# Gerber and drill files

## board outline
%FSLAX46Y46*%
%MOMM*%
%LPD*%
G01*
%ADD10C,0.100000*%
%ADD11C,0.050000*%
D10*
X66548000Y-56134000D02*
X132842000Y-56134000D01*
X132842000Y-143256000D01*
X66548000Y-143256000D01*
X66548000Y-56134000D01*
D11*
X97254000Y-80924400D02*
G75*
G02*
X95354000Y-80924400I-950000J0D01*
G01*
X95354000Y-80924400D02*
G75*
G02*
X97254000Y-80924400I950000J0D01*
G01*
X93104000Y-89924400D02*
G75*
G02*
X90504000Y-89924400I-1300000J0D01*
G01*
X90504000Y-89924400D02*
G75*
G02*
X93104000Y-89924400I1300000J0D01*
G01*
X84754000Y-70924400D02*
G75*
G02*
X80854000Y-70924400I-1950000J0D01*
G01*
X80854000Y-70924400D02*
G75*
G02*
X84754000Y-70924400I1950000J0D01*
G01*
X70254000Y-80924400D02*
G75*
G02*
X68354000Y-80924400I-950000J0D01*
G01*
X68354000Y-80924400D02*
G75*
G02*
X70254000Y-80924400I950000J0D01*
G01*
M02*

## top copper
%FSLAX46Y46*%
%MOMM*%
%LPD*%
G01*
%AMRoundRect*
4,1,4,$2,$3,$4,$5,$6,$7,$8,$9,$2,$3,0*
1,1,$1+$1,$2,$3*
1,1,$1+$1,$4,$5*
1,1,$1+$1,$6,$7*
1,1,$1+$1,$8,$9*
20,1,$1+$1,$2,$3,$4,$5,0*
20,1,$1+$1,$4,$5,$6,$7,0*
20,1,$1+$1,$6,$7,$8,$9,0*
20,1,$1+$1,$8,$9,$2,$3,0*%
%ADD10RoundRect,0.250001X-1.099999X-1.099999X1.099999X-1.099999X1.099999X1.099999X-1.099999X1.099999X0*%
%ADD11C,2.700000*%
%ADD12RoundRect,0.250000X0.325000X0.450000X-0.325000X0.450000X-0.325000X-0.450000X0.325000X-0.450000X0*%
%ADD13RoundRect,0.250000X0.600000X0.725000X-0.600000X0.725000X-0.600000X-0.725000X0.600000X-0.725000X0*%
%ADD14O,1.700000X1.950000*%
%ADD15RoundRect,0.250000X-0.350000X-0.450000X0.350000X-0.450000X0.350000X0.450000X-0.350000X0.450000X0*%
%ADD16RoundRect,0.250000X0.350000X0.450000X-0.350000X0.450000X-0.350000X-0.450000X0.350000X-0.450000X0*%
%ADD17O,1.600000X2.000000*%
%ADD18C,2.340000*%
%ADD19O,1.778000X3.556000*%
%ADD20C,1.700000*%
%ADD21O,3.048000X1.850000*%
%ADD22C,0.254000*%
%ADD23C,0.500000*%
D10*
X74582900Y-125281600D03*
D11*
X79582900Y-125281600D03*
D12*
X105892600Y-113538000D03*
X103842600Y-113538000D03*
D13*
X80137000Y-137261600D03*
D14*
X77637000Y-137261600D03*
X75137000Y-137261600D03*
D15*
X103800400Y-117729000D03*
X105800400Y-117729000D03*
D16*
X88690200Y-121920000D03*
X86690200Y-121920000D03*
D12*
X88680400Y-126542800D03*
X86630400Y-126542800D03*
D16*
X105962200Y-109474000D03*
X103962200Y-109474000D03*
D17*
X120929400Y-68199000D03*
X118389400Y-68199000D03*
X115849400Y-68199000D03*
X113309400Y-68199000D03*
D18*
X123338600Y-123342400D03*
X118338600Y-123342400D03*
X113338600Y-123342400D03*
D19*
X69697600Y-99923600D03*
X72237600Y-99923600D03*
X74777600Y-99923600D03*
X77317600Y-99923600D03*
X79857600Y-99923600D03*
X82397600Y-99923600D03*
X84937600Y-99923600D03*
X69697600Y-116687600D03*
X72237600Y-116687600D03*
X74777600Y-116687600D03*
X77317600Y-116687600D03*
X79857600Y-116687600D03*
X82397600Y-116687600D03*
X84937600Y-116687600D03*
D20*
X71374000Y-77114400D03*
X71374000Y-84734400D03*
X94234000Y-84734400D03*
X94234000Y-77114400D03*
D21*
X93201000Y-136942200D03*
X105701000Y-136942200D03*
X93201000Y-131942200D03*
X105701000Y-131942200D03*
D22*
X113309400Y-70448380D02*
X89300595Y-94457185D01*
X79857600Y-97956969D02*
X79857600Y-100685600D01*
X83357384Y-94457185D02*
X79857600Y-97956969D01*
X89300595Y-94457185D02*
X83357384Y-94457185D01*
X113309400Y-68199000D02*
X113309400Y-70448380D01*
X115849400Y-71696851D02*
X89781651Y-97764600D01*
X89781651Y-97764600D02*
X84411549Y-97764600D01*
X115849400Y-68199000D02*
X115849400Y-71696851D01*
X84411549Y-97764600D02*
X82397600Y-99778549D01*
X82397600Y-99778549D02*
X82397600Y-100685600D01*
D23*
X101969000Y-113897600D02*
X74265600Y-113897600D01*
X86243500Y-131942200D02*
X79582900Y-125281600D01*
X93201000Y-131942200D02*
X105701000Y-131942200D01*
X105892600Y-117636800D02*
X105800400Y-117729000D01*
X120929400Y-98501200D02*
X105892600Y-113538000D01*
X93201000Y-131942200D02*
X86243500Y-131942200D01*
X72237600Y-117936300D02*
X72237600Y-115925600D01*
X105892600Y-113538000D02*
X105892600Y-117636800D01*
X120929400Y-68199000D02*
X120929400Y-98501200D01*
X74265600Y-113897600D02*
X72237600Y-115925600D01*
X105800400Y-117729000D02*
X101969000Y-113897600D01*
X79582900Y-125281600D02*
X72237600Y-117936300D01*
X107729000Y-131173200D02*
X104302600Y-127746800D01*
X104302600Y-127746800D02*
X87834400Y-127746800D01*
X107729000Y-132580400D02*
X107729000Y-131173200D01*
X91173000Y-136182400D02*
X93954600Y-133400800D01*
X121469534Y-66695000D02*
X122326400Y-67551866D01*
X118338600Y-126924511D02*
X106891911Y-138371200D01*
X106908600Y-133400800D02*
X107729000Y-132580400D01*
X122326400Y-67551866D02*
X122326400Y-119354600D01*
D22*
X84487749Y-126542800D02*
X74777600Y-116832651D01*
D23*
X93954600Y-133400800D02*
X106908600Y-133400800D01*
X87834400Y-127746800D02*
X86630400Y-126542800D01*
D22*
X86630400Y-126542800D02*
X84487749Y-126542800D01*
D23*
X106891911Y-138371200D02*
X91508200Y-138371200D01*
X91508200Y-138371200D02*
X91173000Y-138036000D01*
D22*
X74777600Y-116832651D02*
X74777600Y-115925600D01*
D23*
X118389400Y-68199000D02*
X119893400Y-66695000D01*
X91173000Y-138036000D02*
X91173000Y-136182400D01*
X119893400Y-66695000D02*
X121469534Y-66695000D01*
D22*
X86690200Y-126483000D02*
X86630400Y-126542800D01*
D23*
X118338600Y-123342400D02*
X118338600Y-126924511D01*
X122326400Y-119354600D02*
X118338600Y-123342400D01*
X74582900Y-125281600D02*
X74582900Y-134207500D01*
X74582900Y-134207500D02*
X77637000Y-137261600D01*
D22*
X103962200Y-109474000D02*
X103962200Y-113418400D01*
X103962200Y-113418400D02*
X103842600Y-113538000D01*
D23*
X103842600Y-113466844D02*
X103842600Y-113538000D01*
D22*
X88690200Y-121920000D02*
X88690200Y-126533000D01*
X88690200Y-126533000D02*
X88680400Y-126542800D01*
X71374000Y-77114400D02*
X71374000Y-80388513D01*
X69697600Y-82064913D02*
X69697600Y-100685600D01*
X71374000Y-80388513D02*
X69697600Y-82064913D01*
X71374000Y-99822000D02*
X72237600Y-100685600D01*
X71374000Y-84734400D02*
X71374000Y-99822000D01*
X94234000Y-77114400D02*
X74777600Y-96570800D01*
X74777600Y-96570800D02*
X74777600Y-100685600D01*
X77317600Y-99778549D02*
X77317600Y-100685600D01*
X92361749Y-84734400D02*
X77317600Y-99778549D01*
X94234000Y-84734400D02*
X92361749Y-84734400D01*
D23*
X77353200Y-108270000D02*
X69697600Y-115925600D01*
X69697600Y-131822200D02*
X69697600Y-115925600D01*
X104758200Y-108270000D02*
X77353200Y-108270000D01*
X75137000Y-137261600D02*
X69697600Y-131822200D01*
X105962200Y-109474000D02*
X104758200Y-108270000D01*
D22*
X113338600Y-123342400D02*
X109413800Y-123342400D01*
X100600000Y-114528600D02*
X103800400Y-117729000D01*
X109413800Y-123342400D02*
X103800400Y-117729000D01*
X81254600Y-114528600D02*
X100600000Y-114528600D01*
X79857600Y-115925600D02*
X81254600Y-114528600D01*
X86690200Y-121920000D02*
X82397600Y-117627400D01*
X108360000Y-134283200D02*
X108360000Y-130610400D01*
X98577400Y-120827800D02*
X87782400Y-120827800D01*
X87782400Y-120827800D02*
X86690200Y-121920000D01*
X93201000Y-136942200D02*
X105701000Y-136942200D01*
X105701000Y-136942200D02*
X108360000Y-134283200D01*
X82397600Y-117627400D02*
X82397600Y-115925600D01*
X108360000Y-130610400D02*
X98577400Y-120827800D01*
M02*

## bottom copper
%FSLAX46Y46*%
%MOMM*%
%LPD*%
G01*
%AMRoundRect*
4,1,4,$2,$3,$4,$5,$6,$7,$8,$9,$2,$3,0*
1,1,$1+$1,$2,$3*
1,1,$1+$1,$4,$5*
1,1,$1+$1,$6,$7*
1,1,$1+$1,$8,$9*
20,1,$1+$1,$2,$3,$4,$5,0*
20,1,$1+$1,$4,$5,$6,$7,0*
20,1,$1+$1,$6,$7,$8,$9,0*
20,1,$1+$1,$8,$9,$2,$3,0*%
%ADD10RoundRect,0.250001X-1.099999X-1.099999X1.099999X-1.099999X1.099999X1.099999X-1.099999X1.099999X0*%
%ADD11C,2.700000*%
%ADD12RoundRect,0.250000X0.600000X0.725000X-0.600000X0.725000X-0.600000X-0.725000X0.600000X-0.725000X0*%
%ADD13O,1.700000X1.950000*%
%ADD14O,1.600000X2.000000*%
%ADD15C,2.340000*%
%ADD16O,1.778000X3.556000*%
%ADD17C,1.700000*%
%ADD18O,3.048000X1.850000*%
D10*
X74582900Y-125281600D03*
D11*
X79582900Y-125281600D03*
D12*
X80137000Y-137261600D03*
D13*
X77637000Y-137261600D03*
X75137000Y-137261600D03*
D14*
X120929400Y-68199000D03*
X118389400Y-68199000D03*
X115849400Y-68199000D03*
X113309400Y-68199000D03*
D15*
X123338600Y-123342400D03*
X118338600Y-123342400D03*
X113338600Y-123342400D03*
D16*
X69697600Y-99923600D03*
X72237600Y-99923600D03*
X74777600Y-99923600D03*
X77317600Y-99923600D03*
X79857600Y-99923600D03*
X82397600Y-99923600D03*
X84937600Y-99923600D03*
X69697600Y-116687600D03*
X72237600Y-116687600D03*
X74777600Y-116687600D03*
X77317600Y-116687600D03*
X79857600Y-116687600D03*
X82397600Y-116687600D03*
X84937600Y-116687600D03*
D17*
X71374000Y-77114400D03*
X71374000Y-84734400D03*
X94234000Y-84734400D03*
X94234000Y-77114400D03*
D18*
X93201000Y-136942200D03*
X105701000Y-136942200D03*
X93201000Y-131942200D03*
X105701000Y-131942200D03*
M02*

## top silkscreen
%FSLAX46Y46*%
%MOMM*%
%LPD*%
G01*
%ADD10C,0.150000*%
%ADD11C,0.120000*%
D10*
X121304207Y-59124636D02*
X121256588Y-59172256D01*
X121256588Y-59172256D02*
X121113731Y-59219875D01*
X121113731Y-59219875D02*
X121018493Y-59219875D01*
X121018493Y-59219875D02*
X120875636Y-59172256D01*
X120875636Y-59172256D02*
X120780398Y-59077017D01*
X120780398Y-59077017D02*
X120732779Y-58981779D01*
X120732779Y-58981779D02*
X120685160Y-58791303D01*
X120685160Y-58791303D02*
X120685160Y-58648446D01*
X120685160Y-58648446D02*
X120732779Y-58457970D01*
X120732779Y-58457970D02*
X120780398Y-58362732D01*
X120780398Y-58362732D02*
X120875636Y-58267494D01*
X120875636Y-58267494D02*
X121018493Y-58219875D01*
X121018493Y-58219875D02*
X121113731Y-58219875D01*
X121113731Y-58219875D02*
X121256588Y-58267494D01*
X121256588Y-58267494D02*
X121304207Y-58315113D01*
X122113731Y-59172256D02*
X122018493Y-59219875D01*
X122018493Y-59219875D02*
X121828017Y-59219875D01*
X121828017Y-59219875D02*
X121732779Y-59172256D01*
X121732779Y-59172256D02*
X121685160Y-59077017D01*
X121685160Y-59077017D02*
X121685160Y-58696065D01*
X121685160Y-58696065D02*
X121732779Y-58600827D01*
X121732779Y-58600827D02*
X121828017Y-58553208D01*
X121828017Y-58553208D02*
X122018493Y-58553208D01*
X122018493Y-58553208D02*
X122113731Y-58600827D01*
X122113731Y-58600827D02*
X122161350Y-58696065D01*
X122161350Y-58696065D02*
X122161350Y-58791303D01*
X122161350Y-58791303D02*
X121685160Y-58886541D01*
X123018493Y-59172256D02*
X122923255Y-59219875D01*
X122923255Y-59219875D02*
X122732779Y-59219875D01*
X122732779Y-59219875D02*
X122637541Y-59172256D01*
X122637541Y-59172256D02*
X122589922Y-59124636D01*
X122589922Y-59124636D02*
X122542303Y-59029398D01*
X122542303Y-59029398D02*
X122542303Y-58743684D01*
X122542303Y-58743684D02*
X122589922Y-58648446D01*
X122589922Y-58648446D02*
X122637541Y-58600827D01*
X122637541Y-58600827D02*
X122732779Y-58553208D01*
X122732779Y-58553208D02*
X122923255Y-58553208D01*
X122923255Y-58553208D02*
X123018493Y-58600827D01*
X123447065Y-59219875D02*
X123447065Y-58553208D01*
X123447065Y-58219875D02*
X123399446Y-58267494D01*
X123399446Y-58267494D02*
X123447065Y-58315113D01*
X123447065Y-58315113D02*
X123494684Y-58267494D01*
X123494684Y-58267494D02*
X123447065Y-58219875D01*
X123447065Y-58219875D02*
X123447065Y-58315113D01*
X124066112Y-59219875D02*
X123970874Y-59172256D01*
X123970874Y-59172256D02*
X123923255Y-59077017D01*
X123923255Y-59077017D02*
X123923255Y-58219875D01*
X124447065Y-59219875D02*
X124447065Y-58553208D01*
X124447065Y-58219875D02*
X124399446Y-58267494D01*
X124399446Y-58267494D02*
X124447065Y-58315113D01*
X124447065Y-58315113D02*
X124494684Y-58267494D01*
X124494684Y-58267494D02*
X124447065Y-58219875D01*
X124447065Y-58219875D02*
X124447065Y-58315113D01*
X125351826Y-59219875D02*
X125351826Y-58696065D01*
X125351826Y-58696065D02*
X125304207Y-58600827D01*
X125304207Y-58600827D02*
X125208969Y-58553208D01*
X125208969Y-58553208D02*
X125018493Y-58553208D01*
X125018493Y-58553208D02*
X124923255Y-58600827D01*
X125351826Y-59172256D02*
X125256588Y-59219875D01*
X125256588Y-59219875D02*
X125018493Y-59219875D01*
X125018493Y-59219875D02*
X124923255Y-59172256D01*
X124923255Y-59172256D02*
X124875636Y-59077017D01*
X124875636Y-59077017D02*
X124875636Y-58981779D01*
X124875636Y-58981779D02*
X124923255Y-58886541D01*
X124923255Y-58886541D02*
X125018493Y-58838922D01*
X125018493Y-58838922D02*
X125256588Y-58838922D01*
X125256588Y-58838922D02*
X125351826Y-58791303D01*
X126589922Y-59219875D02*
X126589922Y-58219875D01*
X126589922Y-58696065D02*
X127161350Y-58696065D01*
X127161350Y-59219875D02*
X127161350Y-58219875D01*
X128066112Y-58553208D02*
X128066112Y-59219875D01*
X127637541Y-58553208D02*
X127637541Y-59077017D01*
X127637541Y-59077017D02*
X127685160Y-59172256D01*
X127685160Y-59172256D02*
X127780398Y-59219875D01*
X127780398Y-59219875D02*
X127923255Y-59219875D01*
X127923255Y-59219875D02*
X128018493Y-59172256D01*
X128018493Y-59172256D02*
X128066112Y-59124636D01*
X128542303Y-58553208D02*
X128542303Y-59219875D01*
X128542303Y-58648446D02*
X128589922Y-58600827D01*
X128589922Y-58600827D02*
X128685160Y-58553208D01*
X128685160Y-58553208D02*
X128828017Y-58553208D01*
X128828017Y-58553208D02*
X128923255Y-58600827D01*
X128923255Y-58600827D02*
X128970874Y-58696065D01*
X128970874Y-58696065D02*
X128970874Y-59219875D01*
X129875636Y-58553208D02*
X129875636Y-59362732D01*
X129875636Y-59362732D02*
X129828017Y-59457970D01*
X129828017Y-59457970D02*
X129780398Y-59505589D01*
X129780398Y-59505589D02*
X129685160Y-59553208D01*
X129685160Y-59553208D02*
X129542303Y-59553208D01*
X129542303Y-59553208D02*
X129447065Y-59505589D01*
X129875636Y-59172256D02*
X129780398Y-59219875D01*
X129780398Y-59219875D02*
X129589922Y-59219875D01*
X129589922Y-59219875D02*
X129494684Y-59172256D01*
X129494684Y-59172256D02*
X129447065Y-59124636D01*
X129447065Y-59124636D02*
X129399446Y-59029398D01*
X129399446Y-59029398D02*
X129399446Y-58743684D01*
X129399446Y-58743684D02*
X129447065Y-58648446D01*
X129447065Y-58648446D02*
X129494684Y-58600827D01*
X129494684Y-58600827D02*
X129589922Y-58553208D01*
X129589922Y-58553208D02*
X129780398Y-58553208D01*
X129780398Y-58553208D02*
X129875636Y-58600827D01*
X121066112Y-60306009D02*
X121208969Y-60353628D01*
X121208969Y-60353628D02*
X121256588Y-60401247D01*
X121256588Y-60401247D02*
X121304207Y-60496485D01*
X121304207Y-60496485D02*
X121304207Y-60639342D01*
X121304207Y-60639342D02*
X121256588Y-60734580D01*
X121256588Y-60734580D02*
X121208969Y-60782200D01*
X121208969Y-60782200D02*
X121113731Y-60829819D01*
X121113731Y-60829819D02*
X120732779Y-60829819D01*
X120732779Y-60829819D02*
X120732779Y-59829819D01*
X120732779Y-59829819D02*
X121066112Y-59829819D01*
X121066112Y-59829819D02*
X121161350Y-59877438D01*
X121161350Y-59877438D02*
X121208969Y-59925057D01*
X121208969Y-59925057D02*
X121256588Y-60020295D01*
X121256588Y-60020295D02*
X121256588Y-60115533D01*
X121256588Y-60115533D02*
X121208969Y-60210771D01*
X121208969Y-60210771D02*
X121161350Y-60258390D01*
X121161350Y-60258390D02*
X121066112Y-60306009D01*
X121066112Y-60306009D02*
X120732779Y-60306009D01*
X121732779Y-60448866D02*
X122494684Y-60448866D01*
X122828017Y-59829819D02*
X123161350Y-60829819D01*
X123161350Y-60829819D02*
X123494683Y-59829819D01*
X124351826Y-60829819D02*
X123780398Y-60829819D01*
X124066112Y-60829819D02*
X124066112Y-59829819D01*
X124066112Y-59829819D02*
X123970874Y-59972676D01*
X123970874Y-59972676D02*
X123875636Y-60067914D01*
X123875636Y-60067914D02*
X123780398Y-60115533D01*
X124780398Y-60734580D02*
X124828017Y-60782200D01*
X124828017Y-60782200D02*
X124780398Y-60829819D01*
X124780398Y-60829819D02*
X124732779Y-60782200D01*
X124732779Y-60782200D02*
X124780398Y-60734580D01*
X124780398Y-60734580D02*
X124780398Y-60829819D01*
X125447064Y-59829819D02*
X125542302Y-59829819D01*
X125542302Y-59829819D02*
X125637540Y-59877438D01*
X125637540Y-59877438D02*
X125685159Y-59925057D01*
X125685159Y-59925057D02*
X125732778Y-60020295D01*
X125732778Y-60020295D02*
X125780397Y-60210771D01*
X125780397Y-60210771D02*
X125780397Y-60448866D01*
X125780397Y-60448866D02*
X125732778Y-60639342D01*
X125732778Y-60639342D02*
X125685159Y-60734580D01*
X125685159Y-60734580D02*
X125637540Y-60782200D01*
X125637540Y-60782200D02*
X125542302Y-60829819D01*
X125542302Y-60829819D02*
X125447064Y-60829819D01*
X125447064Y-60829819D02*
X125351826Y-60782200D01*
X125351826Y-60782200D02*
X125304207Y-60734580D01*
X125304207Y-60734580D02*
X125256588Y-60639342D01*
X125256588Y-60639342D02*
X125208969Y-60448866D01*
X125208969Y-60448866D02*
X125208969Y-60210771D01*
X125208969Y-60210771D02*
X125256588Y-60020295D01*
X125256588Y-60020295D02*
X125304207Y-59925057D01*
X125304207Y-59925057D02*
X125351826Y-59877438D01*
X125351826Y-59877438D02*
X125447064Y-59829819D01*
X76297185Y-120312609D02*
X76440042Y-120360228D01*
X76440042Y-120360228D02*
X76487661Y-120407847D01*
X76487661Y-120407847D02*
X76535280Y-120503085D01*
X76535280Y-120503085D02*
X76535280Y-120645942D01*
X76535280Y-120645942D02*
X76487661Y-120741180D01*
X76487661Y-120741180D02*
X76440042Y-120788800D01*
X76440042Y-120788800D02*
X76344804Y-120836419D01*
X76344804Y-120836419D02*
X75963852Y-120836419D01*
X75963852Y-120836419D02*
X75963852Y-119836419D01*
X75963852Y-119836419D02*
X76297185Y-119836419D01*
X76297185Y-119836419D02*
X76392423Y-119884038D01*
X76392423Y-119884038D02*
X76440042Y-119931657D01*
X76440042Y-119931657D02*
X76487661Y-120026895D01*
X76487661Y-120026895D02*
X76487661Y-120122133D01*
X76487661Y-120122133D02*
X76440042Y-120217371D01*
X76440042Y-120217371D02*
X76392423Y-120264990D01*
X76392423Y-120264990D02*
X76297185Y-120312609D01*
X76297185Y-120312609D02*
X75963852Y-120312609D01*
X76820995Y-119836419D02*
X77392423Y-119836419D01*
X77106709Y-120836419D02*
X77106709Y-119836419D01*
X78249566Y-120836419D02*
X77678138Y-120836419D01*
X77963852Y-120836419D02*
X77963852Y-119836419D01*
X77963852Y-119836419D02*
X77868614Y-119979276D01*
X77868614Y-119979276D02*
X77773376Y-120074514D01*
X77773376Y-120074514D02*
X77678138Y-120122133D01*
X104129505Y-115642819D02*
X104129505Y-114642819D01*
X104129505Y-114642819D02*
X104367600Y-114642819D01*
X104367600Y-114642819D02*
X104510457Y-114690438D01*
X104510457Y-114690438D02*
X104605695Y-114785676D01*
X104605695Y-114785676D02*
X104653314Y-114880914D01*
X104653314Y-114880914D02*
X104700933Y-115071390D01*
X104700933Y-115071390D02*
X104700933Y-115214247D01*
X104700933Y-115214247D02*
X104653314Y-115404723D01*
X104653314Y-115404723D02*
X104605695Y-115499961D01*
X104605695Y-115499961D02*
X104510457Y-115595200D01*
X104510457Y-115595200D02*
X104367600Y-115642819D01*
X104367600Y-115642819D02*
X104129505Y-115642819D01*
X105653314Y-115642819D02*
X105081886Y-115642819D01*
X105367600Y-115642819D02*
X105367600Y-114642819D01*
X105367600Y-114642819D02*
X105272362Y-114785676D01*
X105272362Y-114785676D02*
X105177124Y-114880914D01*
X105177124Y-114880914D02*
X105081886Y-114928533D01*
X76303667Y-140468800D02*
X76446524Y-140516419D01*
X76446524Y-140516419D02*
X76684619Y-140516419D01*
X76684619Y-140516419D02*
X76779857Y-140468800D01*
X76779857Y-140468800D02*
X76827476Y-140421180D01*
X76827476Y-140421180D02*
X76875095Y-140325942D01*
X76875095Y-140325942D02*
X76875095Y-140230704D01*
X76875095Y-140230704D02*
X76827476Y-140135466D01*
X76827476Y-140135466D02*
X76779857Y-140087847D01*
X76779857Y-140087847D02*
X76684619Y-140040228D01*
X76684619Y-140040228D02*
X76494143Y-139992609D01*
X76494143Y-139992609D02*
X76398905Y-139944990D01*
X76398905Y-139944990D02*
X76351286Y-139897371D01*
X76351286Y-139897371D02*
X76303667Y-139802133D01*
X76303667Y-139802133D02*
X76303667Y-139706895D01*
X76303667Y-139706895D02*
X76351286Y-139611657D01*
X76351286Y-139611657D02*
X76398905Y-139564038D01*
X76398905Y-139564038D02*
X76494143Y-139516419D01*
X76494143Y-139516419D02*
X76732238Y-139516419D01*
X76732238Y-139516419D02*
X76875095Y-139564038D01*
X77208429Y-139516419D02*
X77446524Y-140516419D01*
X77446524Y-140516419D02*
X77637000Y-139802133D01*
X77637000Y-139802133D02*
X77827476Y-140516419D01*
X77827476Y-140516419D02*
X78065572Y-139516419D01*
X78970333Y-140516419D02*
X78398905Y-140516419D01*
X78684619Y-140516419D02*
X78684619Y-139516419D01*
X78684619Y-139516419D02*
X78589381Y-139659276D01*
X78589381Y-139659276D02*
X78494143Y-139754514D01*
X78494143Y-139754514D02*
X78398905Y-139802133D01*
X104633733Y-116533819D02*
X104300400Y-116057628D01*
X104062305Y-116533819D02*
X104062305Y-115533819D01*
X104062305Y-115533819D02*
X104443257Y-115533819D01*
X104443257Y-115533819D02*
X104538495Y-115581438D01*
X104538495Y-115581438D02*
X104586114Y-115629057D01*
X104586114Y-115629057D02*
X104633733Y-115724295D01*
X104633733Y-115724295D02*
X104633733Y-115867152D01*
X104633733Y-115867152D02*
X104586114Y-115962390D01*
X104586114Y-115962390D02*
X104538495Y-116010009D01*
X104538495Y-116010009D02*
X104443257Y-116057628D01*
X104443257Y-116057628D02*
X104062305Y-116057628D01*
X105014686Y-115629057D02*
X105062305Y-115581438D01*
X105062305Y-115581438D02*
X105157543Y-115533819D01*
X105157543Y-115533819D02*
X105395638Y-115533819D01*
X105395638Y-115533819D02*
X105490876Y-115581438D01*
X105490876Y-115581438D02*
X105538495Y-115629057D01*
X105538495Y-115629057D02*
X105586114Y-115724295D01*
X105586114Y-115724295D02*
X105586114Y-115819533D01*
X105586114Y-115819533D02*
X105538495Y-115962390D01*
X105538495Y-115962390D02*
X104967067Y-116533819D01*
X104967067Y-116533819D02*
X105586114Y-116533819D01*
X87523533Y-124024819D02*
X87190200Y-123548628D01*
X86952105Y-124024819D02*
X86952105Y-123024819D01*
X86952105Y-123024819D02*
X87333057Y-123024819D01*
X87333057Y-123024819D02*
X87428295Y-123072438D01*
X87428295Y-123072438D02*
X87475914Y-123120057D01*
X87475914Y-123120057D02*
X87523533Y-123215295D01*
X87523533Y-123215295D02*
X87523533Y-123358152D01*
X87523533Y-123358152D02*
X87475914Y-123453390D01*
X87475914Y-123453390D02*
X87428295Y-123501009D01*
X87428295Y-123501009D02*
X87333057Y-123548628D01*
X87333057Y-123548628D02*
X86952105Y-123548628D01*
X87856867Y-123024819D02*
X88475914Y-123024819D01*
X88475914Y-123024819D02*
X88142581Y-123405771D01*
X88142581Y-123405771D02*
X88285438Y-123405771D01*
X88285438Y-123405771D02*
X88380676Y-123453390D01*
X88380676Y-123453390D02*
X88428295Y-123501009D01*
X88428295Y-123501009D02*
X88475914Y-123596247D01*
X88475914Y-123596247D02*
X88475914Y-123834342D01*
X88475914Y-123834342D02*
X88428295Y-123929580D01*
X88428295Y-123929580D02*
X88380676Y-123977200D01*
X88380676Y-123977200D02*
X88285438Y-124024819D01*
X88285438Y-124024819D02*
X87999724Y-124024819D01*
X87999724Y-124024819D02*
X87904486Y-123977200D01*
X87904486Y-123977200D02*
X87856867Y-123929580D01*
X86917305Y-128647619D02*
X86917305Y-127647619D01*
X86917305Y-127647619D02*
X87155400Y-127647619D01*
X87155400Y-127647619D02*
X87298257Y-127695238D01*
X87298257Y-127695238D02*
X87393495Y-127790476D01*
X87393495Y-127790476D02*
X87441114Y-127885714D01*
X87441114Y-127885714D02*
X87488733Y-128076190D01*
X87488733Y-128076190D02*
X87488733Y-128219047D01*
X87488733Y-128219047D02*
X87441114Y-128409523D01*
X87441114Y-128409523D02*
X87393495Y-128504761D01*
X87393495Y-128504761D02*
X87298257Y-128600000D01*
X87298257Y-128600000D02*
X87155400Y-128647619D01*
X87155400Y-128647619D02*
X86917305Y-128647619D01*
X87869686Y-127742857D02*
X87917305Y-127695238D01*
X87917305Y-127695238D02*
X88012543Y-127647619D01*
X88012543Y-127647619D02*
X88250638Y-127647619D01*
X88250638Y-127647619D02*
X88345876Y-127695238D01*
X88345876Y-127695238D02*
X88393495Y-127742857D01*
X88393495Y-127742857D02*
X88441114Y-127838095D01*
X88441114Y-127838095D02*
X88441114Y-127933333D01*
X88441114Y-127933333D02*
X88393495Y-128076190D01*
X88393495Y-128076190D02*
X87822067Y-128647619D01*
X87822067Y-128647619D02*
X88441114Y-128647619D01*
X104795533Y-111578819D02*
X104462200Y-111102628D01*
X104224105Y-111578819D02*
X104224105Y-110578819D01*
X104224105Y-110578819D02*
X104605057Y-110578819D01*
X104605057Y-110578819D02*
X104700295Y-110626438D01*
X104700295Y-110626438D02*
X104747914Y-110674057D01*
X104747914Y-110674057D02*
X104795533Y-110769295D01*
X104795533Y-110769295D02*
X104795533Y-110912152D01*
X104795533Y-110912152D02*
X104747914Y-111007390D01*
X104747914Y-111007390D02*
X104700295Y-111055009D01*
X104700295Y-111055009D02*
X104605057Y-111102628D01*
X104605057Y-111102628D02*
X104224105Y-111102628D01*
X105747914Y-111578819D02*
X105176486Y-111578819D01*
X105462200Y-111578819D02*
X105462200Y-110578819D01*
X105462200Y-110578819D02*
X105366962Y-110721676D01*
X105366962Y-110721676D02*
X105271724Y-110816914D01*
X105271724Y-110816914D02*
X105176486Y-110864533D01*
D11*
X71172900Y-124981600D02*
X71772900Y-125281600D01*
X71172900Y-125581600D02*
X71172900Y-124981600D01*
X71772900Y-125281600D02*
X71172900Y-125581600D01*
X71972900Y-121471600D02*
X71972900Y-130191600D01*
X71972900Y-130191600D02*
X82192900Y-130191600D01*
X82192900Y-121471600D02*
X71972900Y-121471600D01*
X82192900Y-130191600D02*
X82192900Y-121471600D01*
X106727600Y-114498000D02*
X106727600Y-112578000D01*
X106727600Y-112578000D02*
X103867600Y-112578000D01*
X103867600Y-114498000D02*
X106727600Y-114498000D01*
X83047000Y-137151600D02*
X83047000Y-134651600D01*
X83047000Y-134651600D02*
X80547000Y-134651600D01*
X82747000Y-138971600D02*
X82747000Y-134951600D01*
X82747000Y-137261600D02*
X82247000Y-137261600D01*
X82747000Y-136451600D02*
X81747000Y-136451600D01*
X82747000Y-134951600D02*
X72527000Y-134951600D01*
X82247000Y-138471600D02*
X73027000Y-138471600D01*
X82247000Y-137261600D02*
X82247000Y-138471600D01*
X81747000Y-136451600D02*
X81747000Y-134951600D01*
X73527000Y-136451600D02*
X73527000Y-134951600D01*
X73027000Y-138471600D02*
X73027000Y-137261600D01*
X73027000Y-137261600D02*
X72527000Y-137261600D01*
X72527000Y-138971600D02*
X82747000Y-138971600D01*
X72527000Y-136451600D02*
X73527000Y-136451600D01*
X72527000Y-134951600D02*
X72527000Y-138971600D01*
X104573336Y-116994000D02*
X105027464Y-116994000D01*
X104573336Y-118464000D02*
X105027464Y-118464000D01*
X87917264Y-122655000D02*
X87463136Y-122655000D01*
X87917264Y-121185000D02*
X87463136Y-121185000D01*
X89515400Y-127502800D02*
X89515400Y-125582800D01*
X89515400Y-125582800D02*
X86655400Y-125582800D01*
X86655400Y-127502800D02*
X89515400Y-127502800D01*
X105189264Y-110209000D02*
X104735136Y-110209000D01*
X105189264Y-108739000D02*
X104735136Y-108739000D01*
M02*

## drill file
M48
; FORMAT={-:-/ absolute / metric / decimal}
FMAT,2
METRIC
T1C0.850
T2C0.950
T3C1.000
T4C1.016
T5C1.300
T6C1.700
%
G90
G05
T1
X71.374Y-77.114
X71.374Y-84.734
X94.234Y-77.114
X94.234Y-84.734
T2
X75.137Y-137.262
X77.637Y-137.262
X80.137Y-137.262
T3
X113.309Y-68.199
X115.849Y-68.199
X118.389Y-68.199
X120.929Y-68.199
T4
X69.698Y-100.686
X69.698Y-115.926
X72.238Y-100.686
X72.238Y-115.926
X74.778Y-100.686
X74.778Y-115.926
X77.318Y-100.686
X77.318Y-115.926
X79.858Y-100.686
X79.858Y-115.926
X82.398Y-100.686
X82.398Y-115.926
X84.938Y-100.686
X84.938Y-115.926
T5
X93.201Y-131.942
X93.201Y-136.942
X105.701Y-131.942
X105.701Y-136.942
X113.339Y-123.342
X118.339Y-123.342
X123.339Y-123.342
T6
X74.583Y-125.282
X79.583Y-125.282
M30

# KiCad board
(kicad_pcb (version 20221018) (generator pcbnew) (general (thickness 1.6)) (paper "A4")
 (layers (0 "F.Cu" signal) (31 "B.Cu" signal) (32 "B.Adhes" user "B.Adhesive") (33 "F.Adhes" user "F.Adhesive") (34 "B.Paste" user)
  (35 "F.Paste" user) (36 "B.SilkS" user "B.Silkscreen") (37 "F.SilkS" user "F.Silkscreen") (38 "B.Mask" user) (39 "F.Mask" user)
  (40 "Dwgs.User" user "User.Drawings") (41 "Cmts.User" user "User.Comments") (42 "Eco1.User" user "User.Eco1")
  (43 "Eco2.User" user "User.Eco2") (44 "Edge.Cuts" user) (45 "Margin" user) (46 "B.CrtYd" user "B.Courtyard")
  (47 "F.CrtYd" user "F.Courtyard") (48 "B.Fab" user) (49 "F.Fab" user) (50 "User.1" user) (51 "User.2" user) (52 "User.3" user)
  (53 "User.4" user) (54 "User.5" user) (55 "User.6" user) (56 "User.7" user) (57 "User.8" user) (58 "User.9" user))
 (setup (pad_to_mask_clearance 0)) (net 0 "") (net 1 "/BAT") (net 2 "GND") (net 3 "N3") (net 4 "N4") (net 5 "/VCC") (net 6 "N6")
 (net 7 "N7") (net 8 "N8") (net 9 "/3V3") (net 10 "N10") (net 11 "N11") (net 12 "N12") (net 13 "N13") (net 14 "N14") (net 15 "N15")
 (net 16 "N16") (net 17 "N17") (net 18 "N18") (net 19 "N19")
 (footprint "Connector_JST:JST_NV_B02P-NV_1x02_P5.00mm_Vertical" (layer "F.Cu") (at 74.5829 125.2816)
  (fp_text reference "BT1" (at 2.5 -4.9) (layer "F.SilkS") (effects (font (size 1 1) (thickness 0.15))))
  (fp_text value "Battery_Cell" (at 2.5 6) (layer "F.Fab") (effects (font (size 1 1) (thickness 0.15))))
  (fp_line (start -3.41 -0.3) (end -2.81 0) (stroke (width 0.12) (type solid)) (layer "F.SilkS"))
  (fp_line (start -3.41 0.3) (end -3.41 -0.3) (stroke (width 0.12) (type solid)) (layer "F.SilkS"))
  (fp_line (start -2.81 0) (end -3.41 0.3) (stroke (width 0.12) (type solid)) (layer "F.SilkS"))
  (fp_line (start -2.61 -3.81) (end -2.61 4.91) (stroke (width 0.12) (type solid)) (layer "F.SilkS"))
  (fp_line (start -2.61 4.91) (end 7.61 4.91) (stroke (width 0.12) (type solid)) (layer "F.SilkS"))
  (fp_line (start 7.61 -3.81) (end -2.61 -3.81) (stroke (width 0.12) (type solid)) (layer "F.SilkS"))
  (fp_line (start 7.61 4.91) (end 7.61 -3.81) (stroke (width 0.12) (type solid)) (layer "F.SilkS"))
  (pad "1" thru_hole roundrect (at 0 0) (size 2.7 2.7) (drill 1.7) (layers "*.Cu" "*.Mask") (roundrect_rratio 0.09259296296) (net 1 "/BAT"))
  (pad "2" thru_hole circle (at 5 0) (size 2.7 2.7) (drill 1.7) (layers "*.Cu" "*.Mask") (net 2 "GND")))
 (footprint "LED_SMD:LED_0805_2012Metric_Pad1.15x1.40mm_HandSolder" (layer "F.Cu") (at 104.8676 113.538 180)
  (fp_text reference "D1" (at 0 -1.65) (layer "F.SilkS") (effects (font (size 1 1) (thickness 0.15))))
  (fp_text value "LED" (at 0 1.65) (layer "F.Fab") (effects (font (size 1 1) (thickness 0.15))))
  (fp_line (start -1.86 -0.96) (end -1.86 0.96) (stroke (width 0.12) (type solid)) (layer "F.SilkS"))
  (fp_line (start -1.86 0.96) (end 1 0.96) (stroke (width 0.12) (type solid)) (layer "F.SilkS"))
  (fp_line (start 1 -0.96) (end -1.86 -0.96) (stroke (width 0.12) (type solid)) (layer "F.SilkS"))
  (pad "1" smd roundrect (at -1.025 0 180) (size 1.15 1.4) (layers "F.Cu" "F.Paste" "F.Mask") (roundrect_rratio 0.2173913043) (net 2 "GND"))
  (pad "2" smd roundrect (at 1.025 0 180) (size 1.15 1.4) (layers "F.Cu" "F.Paste" "F.Mask") (roundrect_rratio 0.2173913043) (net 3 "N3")))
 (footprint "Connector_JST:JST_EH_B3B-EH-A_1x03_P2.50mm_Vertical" (layer "F.Cu") (at 80.137 137.2616 180)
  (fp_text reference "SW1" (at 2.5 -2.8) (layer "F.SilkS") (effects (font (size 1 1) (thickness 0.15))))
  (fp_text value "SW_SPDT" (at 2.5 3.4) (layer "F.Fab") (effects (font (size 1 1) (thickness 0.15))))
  (fp_line (start -2.91 0.11) (end -2.91 2.61) (stroke (width 0.12) (type solid)) (layer "F.SilkS"))
  (fp_line (start -2.91 2.61) (end -0.41 2.61) (stroke (width 0.12) (type solid)) (layer "F.SilkS"))
  (fp_line (start -2.61 -1.71) (end -2.61 2.31) (stroke (width 0.12) (type solid)) (layer "F.SilkS"))
  (fp_line (start -2.61 0) (end -2.11 0) (stroke (width 0.12) (type solid)) (layer "F.SilkS"))
  (fp_line (start -2.61 0.81) (end -1.61 0.81) (stroke (width 0.12) (type solid)) (layer "F.SilkS"))
  (fp_line (start -2.61 2.31) (end 7.61 2.31) (stroke (width 0.12) (type solid)) (layer "F.SilkS"))
  (fp_line (start -2.11 -1.21) (end 7.11 -1.21) (stroke (width 0.12) (type solid)) (layer "F.SilkS"))
  (fp_line (start -2.11 0) (end -2.11 -1.21) (stroke (width 0.12) (type solid)) (layer "F.SilkS"))
  (fp_line (start -1.61 0.81) (end -1.61 2.31) (stroke (width 0.12) (type solid)) (layer "F.SilkS"))
  (fp_line (start 6.61 0.81) (end 6.61 2.31) (stroke (width 0.12) (type solid)) (layer "F.SilkS"))
  (fp_line (start 7.11 -1.21) (end 7.11 0) (stroke (width 0.12) (type solid)) (layer "F.SilkS"))
  (fp_line (start 7.11 0) (end 7.61 0) (stroke (width 0.12) (type solid)) (layer "F.SilkS"))
  (fp_line (start 7.61 -1.71) (end -2.61 -1.71) (stroke (width 0.12) (type solid)) (layer "F.SilkS"))
  (fp_line (start 7.61 0.81) (end 6.61 0.81) (stroke (width 0.12) (type solid)) (layer "F.SilkS"))
  (fp_line (start 7.61 2.31) (end 7.61 -1.71) (stroke (width 0.12) (type solid)) (layer "F.SilkS"))
  (pad "1" thru_hole roundrect (at 0 0 180) (size 1.7 1.95) (drill 0.95) (layers "*.Cu" "*.Mask") (roundrect_rratio 0.1470588235)
   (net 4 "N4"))
  (pad "2" thru_hole oval (at 2.5 0 180) (size 1.7 1.95) (drill 0.95) (layers "*.Cu" "*.Mask") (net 1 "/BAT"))
  (pad "3" thru_hole oval (at 5 0 180) (size 1.7 1.95) (drill 0.95) (layers "*.Cu" "*.Mask") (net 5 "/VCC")))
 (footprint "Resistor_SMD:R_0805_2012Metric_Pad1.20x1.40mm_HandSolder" (layer "F.Cu") (at 104.8004 117.729)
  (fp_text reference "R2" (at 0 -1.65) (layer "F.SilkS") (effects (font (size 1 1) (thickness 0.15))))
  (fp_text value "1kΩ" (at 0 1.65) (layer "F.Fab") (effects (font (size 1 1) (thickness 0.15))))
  (fp_line (start -0.227064 -0.735) (end 0.227064 -0.735) (stroke (width 0.12) (type solid)) (layer "F.SilkS"))
  (fp_line (start -0.227064 0.735) (end 0.227064 0.735) (stroke (width 0.12) (type solid)) (layer "F.SilkS"))
  (pad "1" smd roundrect (at -1 0) (size 1.2 1.4) (layers "F.Cu" "F.Paste" "F.Mask") (roundrect_rratio 0.2083333333) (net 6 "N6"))
  (pad "2" smd roundrect (at 1 0) (size 1.2 1.4) (layers "F.Cu" "F.Paste" "F.Mask") (roundrect_rratio 0.2083333333) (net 2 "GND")))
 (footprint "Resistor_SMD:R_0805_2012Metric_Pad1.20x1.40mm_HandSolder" (layer "F.Cu") (at 87.6902 121.92 180)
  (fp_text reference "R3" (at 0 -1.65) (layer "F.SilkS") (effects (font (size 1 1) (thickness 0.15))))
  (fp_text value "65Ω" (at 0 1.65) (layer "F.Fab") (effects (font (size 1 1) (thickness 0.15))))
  (fp_line (start -0.227064 -0.735) (end 0.227064 -0.735) (stroke (width 0.12) (type solid)) (layer "F.SilkS"))
  (fp_line (start -0.227064 0.735) (end 0.227064 0.735) (stroke (width 0.12) (type solid)) (layer "F.SilkS"))
  (pad "1" smd roundrect (at -1 0 180) (size 1.2 1.4) (layers "F.Cu" "F.Paste" "F.Mask") (roundrect_rratio 0.2083333333) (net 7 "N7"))
  (pad "2" smd roundrect (at 1 0 180) (size 1.2 1.4) (layers "F.Cu" "F.Paste" "F.Mask") (roundrect_rratio 0.2083333333) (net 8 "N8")))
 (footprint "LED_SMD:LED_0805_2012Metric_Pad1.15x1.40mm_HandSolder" (layer "F.Cu") (at 87.6554 126.5428 180)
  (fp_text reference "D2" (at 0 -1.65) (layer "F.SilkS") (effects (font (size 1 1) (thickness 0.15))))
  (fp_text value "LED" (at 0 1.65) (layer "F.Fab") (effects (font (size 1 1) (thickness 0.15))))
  (fp_line (start -1.86 -0.96) (end -1.86 0.96) (stroke (width 0.12) (type solid)) (layer "F.SilkS"))
  (fp_line (start -1.86 0.96) (end 1 0.96) (stroke (width 0.12) (type solid)) (layer "F.SilkS"))
  (fp_line (start 1 -0.96) (end -1.86 -0.96) (stroke (width 0.12) (type solid)) (layer "F.SilkS"))
  (pad "1" smd roundrect (at -1.025 0 180) (size 1.15 1.4) (layers "F.Cu" "F.Paste" "F.Mask") (roundrect_rratio 0.2173913043) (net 7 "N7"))
  (pad "2" smd roundrect (at 1.025 0 180) (size 1.15 1.4) (layers "F.Cu" "F.Paste" "F.Mask") (roundrect_rratio 0.2173913043) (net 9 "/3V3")))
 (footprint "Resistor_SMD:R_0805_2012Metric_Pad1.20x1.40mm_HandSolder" (layer "F.Cu") (at 104.9622 109.474 180)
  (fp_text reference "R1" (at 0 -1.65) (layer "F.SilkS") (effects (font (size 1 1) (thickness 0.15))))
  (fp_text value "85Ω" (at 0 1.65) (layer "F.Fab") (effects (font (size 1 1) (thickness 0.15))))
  (fp_line (start -0.227064 -0.735) (end 0.227064 -0.735) (stroke (width 0.12) (type solid)) (layer "F.SilkS"))
  (fp_line (start -0.227064 0.735) (end 0.227064 0.735) (stroke (width 0.12) (type solid)) (layer "F.SilkS"))
  (pad "1" smd roundrect (at -1 0 180) (size 1.2 1.4) (layers "F.Cu" "F.Paste" "F.Mask") (roundrect_rratio 0.2083333333) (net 5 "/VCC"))
  (pad "2" smd roundrect (at 1 0 180) (size 1.2 1.4) (layers "F.Cu" "F.Paste" "F.Mask") (roundrect_rratio 0.2083333333) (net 3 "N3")))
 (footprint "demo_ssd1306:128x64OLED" (layer "B.Cu") (at 117.3094 78.799 180)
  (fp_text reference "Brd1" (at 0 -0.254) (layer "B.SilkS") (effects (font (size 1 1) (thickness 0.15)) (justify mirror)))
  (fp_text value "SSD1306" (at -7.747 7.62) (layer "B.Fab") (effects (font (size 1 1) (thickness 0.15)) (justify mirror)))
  (pad "1" thru_hole oval (at -3.62 10.6 90) (size 2 1.6) (drill 1) (layers "*.Cu" "*.Mask") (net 2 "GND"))
  (pad "2" thru_hole oval (at -1.08 10.6 90) (size 2 1.6) (drill 1) (layers "*.Cu" "*.Mask") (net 9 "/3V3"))
  (pad "3" thru_hole oval (at 1.46 10.6 90) (size 2 1.6) (drill 1) (layers "*.Cu" "*.Mask") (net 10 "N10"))
  (pad "4" thru_hole oval (at 4 10.6 90) (size 2 1.6) (drill 1) (layers "*.Cu" "*.Mask") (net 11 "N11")))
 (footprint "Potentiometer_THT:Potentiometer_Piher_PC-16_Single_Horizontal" (layer "B.Cu") (at 123.3386 123.3424 -90)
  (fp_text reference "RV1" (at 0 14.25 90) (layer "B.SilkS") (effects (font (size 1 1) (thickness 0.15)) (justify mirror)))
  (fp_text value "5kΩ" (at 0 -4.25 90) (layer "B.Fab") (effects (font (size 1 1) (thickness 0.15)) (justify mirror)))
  (pad "1" thru_hole circle (at 0 0 270) (size 2.34 2.34) (drill 1.3) (layers "*.Cu" "*.Mask") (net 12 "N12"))
  (pad "2" thru_hole circle (at 0 5 270) (size 2.34 2.34) (drill 1.3) (layers "*.Cu" "*.Mask") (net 9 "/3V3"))
  (pad "3" thru_hole circle (at 0 10 270) (size 2.34 2.34) (drill 1.3) (layers "*.Cu" "*.Mask") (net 6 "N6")))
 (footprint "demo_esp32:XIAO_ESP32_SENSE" (layer "B.Cu") (at 77.3176 108.3056 -90)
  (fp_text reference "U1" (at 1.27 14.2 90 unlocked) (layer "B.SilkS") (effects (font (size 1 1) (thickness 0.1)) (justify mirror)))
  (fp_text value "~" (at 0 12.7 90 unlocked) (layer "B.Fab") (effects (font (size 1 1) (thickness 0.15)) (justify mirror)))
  (pad "1" thru_hole oval (at -7.62 7.62 270) (size 3.556 1.778) (drill 1.016 (offset -0.762 0)) (layers "*.Cu" "*.Mask") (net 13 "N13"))
  (pad "2" thru_hole oval (at -7.62 5.08 270) (size 3.556 1.778) (drill 1.016 (offset -0.762 0)) (layers "*.Cu" "*.Mask") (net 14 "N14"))
  (pad "3" thru_hole oval (at -7.62 2.54 270) (size 3.556 1.778) (drill 1.016 (offset -0.762 0)) (layers "*.Cu" "*.Mask") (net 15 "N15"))
  (pad "4" thru_hole oval (at -7.62 0 270) (size 3.556 1.778) (drill 1.016 (offset -0.762 0)) (layers "*.Cu" "*.Mask") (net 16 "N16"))
  (pad "5" thru_hole oval (at -7.62 -2.54 270) (size 3.556 1.778) (drill 1.016 (offset -0.762 0)) (layers "*.Cu" "*.Mask") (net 11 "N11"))
  (pad "6" thru_hole oval (at -7.62 -5.08 270) (size 3.556 1.778) (drill 1.016 (offset -0.762 0)) (layers "*.Cu" "*.Mask") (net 10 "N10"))
  (pad "7" thru_hole oval (at -7.62 -7.62 270) (size 3.556 1.778) (drill 1.016 (offset -0.762 0)) (layers "*.Cu" "*.Mask") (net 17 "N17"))
  (pad "8" thru_hole oval (at 7.62 7.62 270) (size 3.556 1.778) (drill 1.016 (offset 0.762 0)) (layers "*.Cu" "*.Mask") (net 5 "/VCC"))
  (pad "9" thru_hole oval (at 7.62 5.08 270) (size 3.556 1.778) (drill 1.016 (offset 0.762 0)) (layers "*.Cu" "*.Mask") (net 2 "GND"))
  (pad "10" thru_hole oval (at 7.62 2.54 270) (size 3.556 1.778) (drill 1.016 (offset 0.762 0)) (layers "*.Cu" "*.Mask") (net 9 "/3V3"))
  (pad "11" thru_hole oval (at 7.62 0 270) (size 3.556 1.778) (drill 1.016 (offset 0.762 0)) (layers "*.Cu" "*.Mask") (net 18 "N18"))
  (pad "12" thru_hole oval (at 7.62 -2.54 270) (size 3.556 1.778) (drill 1.016 (offset 0.762 0)) (layers "*.Cu" "*.Mask") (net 6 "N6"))
  (pad "13" thru_hole oval (at 7.62 -5.08 270) (size 3.556 1.778) (drill 1.016 (offset 0.762 0)) (layers "*.Cu" "*.Mask") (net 8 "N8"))
  (pad "14" thru_hole oval (at 7.62 -7.62 270) (size 3.556 1.778) (drill 1.016 (offset 0.762 0)) (layers "*.Cu" "*.Mask") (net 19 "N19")))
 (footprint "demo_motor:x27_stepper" (layer "B.Cu") (at 80.264 91.0844 180)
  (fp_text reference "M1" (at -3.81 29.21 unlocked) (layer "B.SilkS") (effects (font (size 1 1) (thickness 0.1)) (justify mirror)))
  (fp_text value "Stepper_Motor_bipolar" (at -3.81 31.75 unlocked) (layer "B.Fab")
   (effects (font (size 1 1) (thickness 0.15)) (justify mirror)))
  (fp_circle (center -16.04 10.16) (end -15.09 10.16) (stroke (width 0.05) (type default)) (fill none) (layer "Edge.Cuts"))
  (fp_circle (center -11.54 1.16) (end -10.24 1.16) (stroke (width 0.05) (type default)) (fill none) (layer "Edge.Cuts"))
  (fp_circle (center -2.54 20.16) (end -0.59 20.16) (stroke (width 0.05) (type default)) (fill none) (layer "Edge.Cuts"))
  (fp_circle (center 10.96 10.16) (end 11.91 10.16) (stroke (width 0.05) (type default)) (fill none) (layer "Edge.Cuts"))
  (pad "1" thru_hole circle (at 8.89 13.97 180) (size 1.7 1.7) (drill 0.85) (layers "*.Cu" "*.Mask") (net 13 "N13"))
  (pad "2" thru_hole circle (at 8.89 6.35 180) (size 1.7 1.7) (drill 0.85) (layers "*.Cu" "*.Mask") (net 14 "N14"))
  (pad "3" thru_hole circle (at -13.97 6.35 180) (size 1.7 1.7) (drill 0.85) (layers "*.Cu" "*.Mask") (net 16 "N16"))
  (pad "4" thru_hole circle (at -13.97 13.97 180) (size 1.7 1.7) (drill 0.85) (layers "*.Cu" "*.Mask") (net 15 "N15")))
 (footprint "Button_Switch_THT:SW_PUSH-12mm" (layer "B.Cu") (at 93.201 136.9422)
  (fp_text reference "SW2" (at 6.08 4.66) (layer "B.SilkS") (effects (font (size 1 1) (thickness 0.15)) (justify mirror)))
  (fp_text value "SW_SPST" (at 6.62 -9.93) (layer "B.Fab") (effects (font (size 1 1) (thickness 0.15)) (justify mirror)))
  (pad "1" thru_hole oval (at 0 0) (size 3.048 1.85) (drill 1.3) (layers "*.Cu" "*.Mask") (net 8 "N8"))
  (pad "1" thru_hole oval (at 12.5 0) (size 3.048 1.85) (drill 1.3) (layers "*.Cu" "*.Mask") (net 8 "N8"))
  (pad "2" thru_hole oval (at 0 -5) (size 3.048 1.85) (drill 1.3) (layers "*.Cu" "*.Mask") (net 2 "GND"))
  (pad "2" thru_hole oval (at 12.5 -5) (size 3.048 1.85) (drill 1.3) (layers "*.Cu" "*.Mask") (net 2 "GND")))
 (gr_rect (start 66.548 56.134) (end 132.842 143.256) (stroke (width 0.1) (type default)) (fill none) (layer "Edge.Cuts"))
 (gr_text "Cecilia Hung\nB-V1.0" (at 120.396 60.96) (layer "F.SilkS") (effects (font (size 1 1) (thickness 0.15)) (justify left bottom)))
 (segment (start 113.3094 70.44838) (end 89.300595 94.457185) (width 0.254) (layer "F.Cu") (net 11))
 (segment (start 79.8576 97.956969) (end 79.8576 100.6856) (width 0.254) (layer "F.Cu") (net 11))
 (segment (start 83.357384 94.457185) (end 79.8576 97.956969) (width 0.254) (layer "F.Cu") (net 11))
 (segment (start 89.300595 94.457185) (end 83.357384 94.457185) (width 0.254) (layer "F.Cu") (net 11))
 (segment (start 113.3094 68.199) (end 113.3094 70.44838) (width 0.254) (layer "F.Cu") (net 11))
 (segment (start 115.8494 71.696851) (end 89.781651 97.7646) (width 0.254) (layer "F.Cu") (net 10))
 (segment (start 89.781651 97.7646) (end 84.411549 97.7646) (width 0.254) (layer "F.Cu") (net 10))
 (segment (start 115.8494 68.199) (end 115.8494 71.696851) (width 0.254) (layer "F.Cu") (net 10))
 (segment (start 84.411549 97.7646) (end 82.3976 99.778549) (width 0.254) (layer "F.Cu") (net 10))
 (segment (start 82.3976 99.778549) (end 82.3976 100.6856) (width 0.254) (layer "F.Cu") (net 10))
 (segment (start 101.969 113.8976) (end 74.2656 113.8976) (width 0.5) (layer "F.Cu") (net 2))
 (segment (start 86.2435 131.9422) (end 79.5829 125.2816) (width 0.5) (layer "F.Cu") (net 2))
 (segment (start 93.201 131.9422) (end 105.701 131.9422) (width 0.5) (layer "F.Cu") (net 2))
 (segment (start 105.8926 117.6368) (end 105.8004 117.729) (width 0.5) (layer "F.Cu") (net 2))
 (segment (start 120.9294 98.5012) (end 105.8926 113.538) (width 0.5) (layer "F.Cu") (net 2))
 (segment (start 93.201 131.9422) (end 86.2435 131.9422) (width 0.5) (layer "F.Cu") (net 2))
 (segment (start 72.2376 117.9363) (end 72.2376 115.9256) (width 0.5) (layer "F.Cu") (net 2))
 (segment (start 105.8926 113.538) (end 105.8926 117.6368) (width 0.5) (layer "F.Cu") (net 2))
 (segment (start 120.9294 68.199) (end 120.9294 98.5012) (width 0.5) (layer "F.Cu") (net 2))
 (segment (start 74.2656 113.8976) (end 72.2376 115.9256) (width 0.5) (layer "F.Cu") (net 2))
 (segment (start 105.8004 117.729) (end 101.969 113.8976) (width 0.5) (layer "F.Cu") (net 2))
 (segment (start 79.5829 125.2816) (end 72.2376 117.9363) (width 0.5) (layer "F.Cu") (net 2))
 (segment (start 107.729 131.1732) (end 104.3026 127.7468) (width 0.5) (layer "F.Cu") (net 9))
 (segment (start 104.3026 127.7468) (end 87.8344 127.7468) (width 0.5) (layer "F.Cu") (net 9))
 (segment (start 107.729 132.5804) (end 107.729 131.1732) (width 0.5) (layer "F.Cu") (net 9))
 (segment (start 91.173 136.1824) (end 93.9546 133.4008) (width 0.5) (layer "F.Cu") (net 9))
 (segment (start 121.469534 66.695) (end 122.3264 67.551866) (width 0.5) (layer "F.Cu") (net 9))
 (segment (start 118.3386 126.924511) (end 106.891911 138.3712) (width 0.5) (layer "F.Cu") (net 9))
 (segment (start 106.9086 133.4008) (end 107.729 132.5804) (width 0.5) (layer "F.Cu") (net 9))
 (segment (start 122.3264 67.551866) (end 122.3264 119.3546) (width 0.5) (layer "F.Cu") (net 9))
 (segment (start 84.487749 126.5428) (end 74.7776 116.832651) (width 0.254) (layer "F.Cu") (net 9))
 (segment (start 93.9546 133.4008) (end 106.9086 133.4008) (width 0.5) (layer "F.Cu") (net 9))
 (segment (start 87.8344 127.7468) (end 86.6304 126.5428) (width 0.5) (layer "F.Cu") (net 9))
 (segment (start 86.6304 126.5428) (end 84.487749 126.5428) (width 0.254) (layer "F.Cu") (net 9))
 (segment (start 106.891911 138.3712) (end 91.5082 138.3712) (width 0.5) (layer "F.Cu") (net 9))
 (segment (start 91.5082 138.3712) (end 91.173 138.036) (width 0.5) (layer "F.Cu") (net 9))
 (segment (start 74.7776 116.832651) (end 74.7776 115.9256) (width 0.254) (layer "F.Cu") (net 9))
 (segment (start 118.3894 68.199) (end 119.8934 66.695) (width 0.5) (layer "F.Cu") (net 9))
 (segment (start 91.173 138.036) (end 91.173 136.1824) (width 0.5) (layer "F.Cu") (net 9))
 (segment (start 119.8934 66.695) (end 121.469534 66.695) (width 0.5) (layer "F.Cu") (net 9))
 (segment (start 86.6902 126.483) (end 86.6304 126.5428) (width 0.254) (layer "F.Cu") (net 9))
 (segment (start 118.3386 123.3424) (end 118.3386 126.924511) (width 0.5) (layer "F.Cu") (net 9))
 (segment (start 122.3264 119.3546) (end 118.3386 123.3424) (width 0.5) (layer "F.Cu") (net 9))
 (segment (start 74.5829 125.2816) (end 74.5829 134.2075) (width 0.5) (layer "F.Cu") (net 1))
 (segment (start 74.5829 134.2075) (end 77.637 137.2616) (width 0.5) (layer "F.Cu") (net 1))
 (segment (start 103.9622 109.474) (end 103.9622 113.4184) (width 0.254) (layer "F.Cu") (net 3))
 (segment (start 103.9622 113.4184) (end 103.8426 113.538) (width 0.254) (layer "F.Cu") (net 3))
 (segment (start 103.8426 113.466844) (end 103.8426 113.538) (width 0.5) (layer "F.Cu") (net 3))
 (segment (start 88.6902 121.92) (end 88.6902 126.533) (width 0.254) (layer "F.Cu") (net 7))
 (segment (start 88.6902 126.533) (end 88.6804 126.5428) (width 0.254) (layer "F.Cu") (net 7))
 (segment (start 71.374 77.1144) (end 71.374 80.388513) (width 0.254) (layer "F.Cu") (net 13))
 (segment (start 69.6976 82.064913) (end 69.6976 100.6856) (width 0.254) (layer "F.Cu") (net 13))
 (segment (start 71.374 80.388513) (end 69.6976 82.064913) (width 0.254) (layer "F.Cu") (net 13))
 (segment (start 71.374 99.822) (end 72.2376 100.6856) (width 0.254) (layer "F.Cu") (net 14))
 (segment (start 71.374 84.7344) (end 71.374 99.822) (width 0.254) (layer "F.Cu") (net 14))
 (segment (start 94.234 77.1144) (end 74.7776 96.5708) (width 0.254) (layer "F.Cu") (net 15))
 (segment (start 74.7776 96.5708) (end 74.7776 100.6856) (width 0.254) (layer "F.Cu") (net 15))
 (segment (start 77.3176 99.778549) (end 77.3176 100.6856) (width 0.254) (layer "F.Cu") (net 16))
 (segment (start 92.361749 84.7344) (end 77.3176 99.778549) (width 0.254) (layer "F.Cu") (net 16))
 (segment (start 94.234 84.7344) (end 92.361749 84.7344) (width 0.254) (layer "F.Cu") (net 16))
 (segment (start 77.3532 108.27) (end 69.6976 115.9256) (width 0.5) (layer "F.Cu") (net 5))
 (segment (start 69.6976 131.8222) (end 69.6976 115.9256) (width 0.5) (layer "F.Cu") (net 5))
 (segment (start 104.7582 108.27) (end 77.3532 108.27) (width 0.5) (layer "F.Cu") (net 5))
 (segment (start 75.137 137.2616) (end 69.6976 131.8222) (width 0.5) (layer "F.Cu") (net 5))
 (segment (start 105.9622 109.474) (end 104.7582 108.27) (width 0.5) (layer "F.Cu") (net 5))
 (segment (start 113.3386 123.3424) (end 109.4138 123.3424) (width 0.254) (layer "F.Cu") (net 6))
 (segment (start 100.6 114.5286) (end 103.8004 117.729) (width 0.254) (layer "F.Cu") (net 6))
 (segment (start 109.4138 123.3424) (end 103.8004 117.729) (width 0.254) (layer "F.Cu") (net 6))
 (segment (start 81.2546 114.5286) (end 100.6 114.5286) (width 0.254) (layer "F.Cu") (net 6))
 (segment (start 79.8576 115.9256) (end 81.2546 114.5286) (width 0.254) (layer "F.Cu") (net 6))
 (segment (start 86.6902 121.92) (end 82.3976 117.6274) (width 0.254) (layer "F.Cu") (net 8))
 (segment (start 108.36 134.2832) (end 108.36 130.6104) (width 0.254) (layer "F.Cu") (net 8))
 (segment (start 98.5774 120.8278) (end 87.7824 120.8278) (width 0.254) (layer "F.Cu") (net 8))
 (segment (start 87.7824 120.8278) (end 86.6902 121.92) (width 0.254) (layer "F.Cu") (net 8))
 (segment (start 93.201 136.9422) (end 105.701 136.9422) (width 0.254) (layer "F.Cu") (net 8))
 (segment (start 105.701 136.9422) (end 108.36 134.2832) (width 0.254) (layer "F.Cu") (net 8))
 (segment (start 82.3976 117.6274) (end 82.3976 115.9256) (width 0.254) (layer "F.Cu") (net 8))
 (segment (start 108.36 130.6104) (end 98.5774 120.8278) (width 0.254) (layer "F.Cu") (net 8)))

